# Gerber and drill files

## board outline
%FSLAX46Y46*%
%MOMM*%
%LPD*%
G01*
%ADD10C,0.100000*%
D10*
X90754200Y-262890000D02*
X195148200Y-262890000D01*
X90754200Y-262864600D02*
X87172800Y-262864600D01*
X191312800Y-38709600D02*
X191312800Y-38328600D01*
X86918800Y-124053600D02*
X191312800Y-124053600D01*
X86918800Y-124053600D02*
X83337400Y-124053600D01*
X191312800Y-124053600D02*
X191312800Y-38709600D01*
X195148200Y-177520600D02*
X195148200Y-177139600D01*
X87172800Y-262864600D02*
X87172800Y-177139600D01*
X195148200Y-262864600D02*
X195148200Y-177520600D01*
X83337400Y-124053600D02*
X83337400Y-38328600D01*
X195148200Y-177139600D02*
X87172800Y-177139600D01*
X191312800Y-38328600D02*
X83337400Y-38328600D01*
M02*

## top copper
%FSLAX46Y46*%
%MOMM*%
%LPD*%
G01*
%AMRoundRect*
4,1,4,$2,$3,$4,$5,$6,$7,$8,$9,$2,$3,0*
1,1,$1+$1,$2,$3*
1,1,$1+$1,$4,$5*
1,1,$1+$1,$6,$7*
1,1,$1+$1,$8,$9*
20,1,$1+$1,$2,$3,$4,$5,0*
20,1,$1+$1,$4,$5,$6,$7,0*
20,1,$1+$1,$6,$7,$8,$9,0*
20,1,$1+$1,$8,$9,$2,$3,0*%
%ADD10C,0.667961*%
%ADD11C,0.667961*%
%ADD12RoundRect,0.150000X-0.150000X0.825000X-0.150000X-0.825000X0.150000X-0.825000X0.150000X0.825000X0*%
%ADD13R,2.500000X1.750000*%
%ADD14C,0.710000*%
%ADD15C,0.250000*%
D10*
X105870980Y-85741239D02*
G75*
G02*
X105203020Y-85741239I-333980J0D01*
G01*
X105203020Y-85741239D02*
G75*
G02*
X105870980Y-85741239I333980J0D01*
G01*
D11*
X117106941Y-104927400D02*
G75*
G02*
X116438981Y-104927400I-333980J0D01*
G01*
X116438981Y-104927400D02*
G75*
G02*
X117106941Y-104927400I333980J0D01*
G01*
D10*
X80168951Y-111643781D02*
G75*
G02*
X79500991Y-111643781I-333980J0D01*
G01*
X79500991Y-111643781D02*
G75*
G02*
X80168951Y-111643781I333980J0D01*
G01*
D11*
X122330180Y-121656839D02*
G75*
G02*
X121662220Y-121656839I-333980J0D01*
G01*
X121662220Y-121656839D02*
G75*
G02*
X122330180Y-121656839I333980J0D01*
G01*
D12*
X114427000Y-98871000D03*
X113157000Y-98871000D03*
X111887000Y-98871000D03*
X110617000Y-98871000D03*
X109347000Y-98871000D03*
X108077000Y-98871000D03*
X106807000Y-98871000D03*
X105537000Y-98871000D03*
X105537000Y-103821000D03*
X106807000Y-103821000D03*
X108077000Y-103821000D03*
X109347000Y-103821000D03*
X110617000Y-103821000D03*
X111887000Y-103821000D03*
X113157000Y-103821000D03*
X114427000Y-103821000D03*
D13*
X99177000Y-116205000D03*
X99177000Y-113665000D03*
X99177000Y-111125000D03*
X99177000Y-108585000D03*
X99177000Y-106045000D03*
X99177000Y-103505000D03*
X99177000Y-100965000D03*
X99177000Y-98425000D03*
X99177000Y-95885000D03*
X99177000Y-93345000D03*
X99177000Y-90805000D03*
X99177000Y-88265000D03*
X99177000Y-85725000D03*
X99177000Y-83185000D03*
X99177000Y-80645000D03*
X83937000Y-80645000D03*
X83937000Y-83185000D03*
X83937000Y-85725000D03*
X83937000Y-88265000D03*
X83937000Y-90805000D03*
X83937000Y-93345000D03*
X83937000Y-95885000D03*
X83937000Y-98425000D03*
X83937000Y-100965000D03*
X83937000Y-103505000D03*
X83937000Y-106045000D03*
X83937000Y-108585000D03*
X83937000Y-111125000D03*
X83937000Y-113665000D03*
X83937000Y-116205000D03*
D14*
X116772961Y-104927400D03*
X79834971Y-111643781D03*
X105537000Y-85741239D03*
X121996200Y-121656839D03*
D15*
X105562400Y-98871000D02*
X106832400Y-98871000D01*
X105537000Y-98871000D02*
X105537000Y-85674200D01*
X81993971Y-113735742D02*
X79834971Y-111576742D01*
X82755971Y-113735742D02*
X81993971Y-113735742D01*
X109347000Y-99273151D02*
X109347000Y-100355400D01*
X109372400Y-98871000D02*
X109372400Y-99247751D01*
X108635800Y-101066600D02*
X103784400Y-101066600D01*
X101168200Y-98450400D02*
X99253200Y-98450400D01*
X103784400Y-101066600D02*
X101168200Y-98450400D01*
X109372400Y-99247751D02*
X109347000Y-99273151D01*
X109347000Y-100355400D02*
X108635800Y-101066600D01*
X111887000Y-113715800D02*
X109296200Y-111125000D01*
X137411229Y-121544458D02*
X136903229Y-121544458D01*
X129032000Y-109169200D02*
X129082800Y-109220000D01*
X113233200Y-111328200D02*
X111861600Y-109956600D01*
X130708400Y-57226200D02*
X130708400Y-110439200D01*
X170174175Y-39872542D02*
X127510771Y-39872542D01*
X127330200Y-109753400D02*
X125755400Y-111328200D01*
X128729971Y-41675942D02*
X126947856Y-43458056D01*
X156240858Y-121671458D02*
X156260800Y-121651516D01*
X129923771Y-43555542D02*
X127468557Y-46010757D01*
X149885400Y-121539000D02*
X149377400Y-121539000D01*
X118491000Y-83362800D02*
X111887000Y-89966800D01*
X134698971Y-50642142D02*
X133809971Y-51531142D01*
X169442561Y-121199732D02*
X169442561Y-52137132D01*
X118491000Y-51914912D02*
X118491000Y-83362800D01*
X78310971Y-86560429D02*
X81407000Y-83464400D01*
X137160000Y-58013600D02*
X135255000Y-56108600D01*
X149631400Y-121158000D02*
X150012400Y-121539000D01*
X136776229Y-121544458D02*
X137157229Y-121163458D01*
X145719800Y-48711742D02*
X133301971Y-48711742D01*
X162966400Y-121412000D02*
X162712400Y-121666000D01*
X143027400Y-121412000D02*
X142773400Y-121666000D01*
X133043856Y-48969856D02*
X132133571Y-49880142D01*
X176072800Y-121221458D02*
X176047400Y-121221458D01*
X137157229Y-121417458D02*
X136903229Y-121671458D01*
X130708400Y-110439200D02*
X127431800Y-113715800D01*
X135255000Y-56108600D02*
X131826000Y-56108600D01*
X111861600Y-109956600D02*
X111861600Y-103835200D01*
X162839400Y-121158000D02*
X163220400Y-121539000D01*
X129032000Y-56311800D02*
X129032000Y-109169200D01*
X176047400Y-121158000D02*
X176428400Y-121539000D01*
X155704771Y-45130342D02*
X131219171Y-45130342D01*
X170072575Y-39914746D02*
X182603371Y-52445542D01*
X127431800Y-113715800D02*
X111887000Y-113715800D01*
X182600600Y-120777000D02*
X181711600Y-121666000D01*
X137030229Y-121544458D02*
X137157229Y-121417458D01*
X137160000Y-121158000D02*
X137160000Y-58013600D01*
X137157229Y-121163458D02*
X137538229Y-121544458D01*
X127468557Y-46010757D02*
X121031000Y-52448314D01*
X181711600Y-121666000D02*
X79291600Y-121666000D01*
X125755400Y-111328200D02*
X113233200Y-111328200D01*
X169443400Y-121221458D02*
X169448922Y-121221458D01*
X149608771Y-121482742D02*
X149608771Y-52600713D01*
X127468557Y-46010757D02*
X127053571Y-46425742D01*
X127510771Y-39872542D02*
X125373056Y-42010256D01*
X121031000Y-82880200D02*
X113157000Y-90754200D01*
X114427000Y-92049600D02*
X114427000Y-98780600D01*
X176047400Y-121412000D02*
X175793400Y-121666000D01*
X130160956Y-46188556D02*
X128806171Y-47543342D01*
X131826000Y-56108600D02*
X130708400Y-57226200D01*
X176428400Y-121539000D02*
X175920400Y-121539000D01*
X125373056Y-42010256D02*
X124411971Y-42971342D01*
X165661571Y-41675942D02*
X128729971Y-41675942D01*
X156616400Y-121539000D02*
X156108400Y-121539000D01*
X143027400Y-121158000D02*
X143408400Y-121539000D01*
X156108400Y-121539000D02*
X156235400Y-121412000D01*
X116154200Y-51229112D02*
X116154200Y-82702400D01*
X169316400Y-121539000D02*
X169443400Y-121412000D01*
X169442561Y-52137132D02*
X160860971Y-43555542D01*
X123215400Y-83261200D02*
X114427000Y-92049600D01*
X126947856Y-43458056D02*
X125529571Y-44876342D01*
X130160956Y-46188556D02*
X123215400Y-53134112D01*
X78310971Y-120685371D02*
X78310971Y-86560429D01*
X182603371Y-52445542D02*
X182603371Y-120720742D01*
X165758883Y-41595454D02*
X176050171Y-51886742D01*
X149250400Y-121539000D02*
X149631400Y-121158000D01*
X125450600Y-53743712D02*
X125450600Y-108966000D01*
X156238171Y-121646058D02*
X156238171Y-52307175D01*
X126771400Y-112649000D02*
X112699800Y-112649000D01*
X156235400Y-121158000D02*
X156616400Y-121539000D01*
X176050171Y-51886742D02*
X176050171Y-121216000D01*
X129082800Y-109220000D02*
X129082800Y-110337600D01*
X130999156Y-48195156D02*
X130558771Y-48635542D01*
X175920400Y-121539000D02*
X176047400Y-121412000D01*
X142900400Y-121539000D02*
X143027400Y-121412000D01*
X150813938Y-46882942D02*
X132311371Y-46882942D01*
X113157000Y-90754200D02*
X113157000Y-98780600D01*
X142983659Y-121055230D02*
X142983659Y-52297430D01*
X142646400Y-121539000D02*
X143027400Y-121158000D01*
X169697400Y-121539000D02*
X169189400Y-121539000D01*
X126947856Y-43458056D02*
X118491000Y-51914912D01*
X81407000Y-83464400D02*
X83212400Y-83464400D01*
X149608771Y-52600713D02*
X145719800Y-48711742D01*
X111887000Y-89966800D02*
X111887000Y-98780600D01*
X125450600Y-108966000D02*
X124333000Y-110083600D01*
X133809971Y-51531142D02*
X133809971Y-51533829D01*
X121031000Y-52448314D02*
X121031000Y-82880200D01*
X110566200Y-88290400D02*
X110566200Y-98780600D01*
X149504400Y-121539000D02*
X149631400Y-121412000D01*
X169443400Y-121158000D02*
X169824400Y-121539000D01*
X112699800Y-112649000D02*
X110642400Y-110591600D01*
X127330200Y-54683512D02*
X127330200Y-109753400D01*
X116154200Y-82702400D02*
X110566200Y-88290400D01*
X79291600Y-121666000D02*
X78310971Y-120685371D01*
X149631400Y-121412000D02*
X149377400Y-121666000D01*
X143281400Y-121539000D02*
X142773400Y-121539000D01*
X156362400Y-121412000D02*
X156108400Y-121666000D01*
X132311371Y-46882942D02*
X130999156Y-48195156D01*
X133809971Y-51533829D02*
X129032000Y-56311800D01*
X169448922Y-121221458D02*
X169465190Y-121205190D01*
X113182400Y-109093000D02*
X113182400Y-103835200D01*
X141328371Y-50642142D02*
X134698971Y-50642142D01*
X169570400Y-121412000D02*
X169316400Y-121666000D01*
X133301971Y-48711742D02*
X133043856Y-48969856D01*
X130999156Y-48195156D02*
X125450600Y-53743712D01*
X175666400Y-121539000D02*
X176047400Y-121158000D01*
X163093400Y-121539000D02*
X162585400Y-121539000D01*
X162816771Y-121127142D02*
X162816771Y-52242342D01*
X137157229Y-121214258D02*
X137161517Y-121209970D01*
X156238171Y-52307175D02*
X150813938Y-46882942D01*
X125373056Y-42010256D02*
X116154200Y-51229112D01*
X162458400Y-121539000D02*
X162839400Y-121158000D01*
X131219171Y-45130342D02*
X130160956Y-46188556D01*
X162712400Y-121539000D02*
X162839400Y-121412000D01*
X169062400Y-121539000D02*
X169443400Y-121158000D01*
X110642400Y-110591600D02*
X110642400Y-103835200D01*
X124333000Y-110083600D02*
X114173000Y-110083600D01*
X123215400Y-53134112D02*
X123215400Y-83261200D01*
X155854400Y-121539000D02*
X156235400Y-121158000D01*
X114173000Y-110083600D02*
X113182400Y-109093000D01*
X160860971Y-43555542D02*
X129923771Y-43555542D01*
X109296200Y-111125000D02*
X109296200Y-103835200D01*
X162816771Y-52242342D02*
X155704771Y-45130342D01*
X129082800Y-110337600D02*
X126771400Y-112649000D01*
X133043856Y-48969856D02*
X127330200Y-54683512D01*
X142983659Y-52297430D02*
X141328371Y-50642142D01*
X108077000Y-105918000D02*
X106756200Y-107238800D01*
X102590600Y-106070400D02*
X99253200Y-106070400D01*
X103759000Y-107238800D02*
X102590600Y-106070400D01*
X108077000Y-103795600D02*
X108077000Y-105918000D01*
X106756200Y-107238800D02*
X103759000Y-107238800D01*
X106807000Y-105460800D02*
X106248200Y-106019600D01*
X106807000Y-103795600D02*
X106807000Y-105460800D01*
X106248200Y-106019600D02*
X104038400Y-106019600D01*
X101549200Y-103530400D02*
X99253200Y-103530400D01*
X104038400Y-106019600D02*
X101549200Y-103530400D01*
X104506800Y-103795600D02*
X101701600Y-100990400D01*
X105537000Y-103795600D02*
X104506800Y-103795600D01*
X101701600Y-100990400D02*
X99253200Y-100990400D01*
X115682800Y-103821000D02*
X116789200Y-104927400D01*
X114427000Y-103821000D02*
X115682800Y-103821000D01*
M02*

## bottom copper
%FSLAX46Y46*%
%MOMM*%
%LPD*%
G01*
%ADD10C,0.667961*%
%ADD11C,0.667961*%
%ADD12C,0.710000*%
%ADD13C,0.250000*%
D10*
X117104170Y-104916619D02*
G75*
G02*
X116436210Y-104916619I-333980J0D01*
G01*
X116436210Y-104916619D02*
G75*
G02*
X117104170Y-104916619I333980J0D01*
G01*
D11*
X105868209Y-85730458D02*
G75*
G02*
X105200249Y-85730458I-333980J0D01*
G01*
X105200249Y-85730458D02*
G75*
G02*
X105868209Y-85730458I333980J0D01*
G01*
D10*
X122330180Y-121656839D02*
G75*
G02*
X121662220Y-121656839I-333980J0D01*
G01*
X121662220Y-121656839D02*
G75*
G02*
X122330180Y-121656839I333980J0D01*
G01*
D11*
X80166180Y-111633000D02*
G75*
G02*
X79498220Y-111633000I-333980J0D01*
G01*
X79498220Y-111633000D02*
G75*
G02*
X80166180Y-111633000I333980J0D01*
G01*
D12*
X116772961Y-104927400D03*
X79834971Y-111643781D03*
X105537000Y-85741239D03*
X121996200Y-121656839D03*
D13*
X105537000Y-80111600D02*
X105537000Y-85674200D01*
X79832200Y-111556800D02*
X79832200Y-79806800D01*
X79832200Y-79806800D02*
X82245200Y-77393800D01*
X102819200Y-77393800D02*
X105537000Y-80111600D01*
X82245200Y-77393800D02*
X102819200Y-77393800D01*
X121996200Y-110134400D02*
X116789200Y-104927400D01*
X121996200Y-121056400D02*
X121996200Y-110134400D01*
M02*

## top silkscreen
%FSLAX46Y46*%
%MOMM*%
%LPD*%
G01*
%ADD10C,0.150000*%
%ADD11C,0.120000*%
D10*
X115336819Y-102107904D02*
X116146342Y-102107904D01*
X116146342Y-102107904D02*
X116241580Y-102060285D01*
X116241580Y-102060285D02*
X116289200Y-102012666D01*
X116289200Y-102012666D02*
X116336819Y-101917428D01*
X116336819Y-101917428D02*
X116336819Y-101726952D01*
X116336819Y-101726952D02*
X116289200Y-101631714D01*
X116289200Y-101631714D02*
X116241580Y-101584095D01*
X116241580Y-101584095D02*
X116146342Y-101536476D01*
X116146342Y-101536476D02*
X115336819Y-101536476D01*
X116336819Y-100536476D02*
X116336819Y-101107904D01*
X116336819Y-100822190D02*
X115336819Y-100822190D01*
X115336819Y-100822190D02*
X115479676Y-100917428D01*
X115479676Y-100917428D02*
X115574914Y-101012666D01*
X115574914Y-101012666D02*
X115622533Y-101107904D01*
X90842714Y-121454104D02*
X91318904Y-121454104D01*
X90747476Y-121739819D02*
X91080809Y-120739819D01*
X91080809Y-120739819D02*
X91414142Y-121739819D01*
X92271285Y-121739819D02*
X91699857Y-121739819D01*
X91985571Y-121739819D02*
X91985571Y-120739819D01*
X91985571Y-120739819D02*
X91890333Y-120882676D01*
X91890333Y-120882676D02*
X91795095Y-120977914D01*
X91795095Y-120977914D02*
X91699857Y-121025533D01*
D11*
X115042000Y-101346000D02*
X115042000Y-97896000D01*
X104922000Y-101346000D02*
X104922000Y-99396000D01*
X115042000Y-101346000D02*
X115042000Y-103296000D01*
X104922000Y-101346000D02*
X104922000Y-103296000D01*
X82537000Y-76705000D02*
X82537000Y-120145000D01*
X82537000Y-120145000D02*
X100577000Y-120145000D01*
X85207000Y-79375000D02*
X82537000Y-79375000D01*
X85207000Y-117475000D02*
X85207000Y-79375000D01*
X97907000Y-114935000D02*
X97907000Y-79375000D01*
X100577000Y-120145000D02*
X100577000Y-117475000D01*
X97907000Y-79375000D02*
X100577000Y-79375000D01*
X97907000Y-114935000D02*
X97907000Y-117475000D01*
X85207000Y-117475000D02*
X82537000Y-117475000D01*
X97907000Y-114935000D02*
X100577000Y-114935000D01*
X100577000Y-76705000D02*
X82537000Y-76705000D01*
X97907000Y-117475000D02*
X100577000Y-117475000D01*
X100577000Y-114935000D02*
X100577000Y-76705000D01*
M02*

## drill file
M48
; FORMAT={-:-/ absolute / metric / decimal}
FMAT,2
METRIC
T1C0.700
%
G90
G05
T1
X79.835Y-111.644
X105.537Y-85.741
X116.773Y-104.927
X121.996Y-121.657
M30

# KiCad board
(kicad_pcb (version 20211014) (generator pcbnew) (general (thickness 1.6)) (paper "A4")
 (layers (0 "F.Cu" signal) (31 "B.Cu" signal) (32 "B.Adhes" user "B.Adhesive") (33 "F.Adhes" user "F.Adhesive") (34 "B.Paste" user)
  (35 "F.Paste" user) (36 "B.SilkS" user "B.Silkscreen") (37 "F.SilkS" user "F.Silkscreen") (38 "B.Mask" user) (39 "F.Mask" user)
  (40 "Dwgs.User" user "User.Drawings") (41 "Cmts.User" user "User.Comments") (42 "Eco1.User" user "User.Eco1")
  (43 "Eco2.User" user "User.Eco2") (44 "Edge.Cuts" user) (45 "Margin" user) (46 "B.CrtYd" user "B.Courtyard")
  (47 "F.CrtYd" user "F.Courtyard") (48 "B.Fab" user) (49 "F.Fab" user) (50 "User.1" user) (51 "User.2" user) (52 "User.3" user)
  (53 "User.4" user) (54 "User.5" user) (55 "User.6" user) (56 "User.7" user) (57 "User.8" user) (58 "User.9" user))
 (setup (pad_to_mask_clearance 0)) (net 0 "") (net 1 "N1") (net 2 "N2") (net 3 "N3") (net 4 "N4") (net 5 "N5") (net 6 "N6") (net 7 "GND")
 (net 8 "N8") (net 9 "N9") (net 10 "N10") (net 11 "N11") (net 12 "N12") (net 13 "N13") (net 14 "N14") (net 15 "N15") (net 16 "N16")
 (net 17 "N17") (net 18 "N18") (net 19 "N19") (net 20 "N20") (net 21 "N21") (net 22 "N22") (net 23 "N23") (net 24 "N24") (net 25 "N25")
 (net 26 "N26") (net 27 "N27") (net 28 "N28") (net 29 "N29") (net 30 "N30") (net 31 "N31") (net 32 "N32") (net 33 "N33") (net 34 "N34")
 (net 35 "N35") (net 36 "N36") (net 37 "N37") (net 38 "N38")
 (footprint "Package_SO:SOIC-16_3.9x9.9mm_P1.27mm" (layer "F.Cu") (at 109.982 101.346 -90)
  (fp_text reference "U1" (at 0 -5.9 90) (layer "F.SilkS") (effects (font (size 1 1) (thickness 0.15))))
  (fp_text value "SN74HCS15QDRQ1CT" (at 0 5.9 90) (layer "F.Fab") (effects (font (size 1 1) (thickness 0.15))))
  (fp_line (start 0 -5.06) (end -3.45 -5.06) (layer "F.SilkS") (width 0.12))
  (fp_line (start 0 5.06) (end -1.95 5.06) (layer "F.SilkS") (width 0.12))
  (fp_line (start 0 -5.06) (end 1.95 -5.06) (layer "F.SilkS") (width 0.12))
  (fp_line (start 0 5.06) (end 1.95 5.06) (layer "F.SilkS") (width 0.12))
  (pad "1" smd roundrect (at -2.475 -4.445 270) (size 1.95 0.6) (layers "F.Cu" "F.Paste" "F.Mask") (roundrect_rratio 0.25) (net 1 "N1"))
  (pad "2" smd roundrect (at -2.475 -3.175 270) (size 1.95 0.6) (layers "F.Cu" "F.Paste" "F.Mask") (roundrect_rratio 0.25) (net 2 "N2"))
  (pad "3" smd roundrect (at -2.475 -1.905 270) (size 1.95 0.6) (layers "F.Cu" "F.Paste" "F.Mask") (roundrect_rratio 0.25) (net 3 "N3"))
  (pad "4" smd roundrect (at -2.475 -0.635 270) (size 1.95 0.6) (layers "F.Cu" "F.Paste" "F.Mask") (roundrect_rratio 0.25) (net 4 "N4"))
  (pad "5" smd roundrect (at -2.475 0.635 270) (size 1.95 0.6) (layers "F.Cu" "F.Paste" "F.Mask") (roundrect_rratio 0.25) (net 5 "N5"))
  (pad "6" smd roundrect (at -2.475 1.905 270) (size 1.95 0.6) (layers "F.Cu" "F.Paste" "F.Mask") (roundrect_rratio 0.25) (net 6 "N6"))
  (pad "7" smd roundrect (at -2.475 3.175 270) (size 1.95 0.6) (layers "F.Cu" "F.Paste" "F.Mask") (roundrect_rratio 0.25) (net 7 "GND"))
  (pad "8" smd roundrect (at -2.475 4.445 270) (size 1.95 0.6) (layers "F.Cu" "F.Paste" "F.Mask") (roundrect_rratio 0.25) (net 7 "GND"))
  (pad "9" smd roundrect (at 2.475 4.445 270) (size 1.95 0.6) (layers "F.Cu" "F.Paste" "F.Mask") (roundrect_rratio 0.25) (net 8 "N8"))
  (pad "10" smd roundrect (at 2.475 3.175 270) (size 1.95 0.6) (layers "F.Cu" "F.Paste" "F.Mask") (roundrect_rratio 0.25) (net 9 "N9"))
  (pad "11" smd roundrect (at 2.475 1.905 270) (size 1.95 0.6) (layers "F.Cu" "F.Paste" "F.Mask") (roundrect_rratio 0.25) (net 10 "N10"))
  (pad "12" smd roundrect (at 2.475 0.635 270) (size 1.95 0.6) (layers "F.Cu" "F.Paste" "F.Mask") (roundrect_rratio 0.25) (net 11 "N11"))
  (pad "13" smd roundrect (at 2.475 -0.635 270) (size 1.95 0.6) (layers "F.Cu" "F.Paste" "F.Mask") (roundrect_rratio 0.25) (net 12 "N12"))
  (pad "14" smd roundrect (at 2.475 -1.905 270) (size 1.95 0.6) (layers "F.Cu" "F.Paste" "F.Mask") (roundrect_rratio 0.25) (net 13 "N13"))
  (pad "15" smd roundrect (at 2.475 -3.175 270) (size 1.95 0.6) (layers "F.Cu" "F.Paste" "F.Mask") (roundrect_rratio 0.25) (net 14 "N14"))
  (pad "16" smd roundrect (at 2.475 -4.445 270) (size 1.95 0.6) (layers "F.Cu" "F.Paste" "F.Mask") (roundrect_rratio 0.25) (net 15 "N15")))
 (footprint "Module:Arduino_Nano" (layer "F.Cu") (at 99.177 116.205 180)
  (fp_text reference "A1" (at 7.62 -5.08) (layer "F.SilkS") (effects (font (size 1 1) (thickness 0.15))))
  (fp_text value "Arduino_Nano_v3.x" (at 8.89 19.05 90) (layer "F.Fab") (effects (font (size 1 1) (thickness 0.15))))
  (fp_line (start 16.64 39.5) (end 16.64 -3.94) (layer "F.SilkS") (width 0.12))
  (fp_line (start 16.64 -3.94) (end -1.4 -3.94) (layer "F.SilkS") (width 0.12))
  (fp_line (start 13.97 36.83) (end 16.64 36.83) (layer "F.SilkS") (width 0.12))
  (fp_line (start 13.97 -1.27) (end 13.97 36.83) (layer "F.SilkS") (width 0.12))
  (fp_line (start 1.27 1.27) (end 1.27 36.83) (layer "F.SilkS") (width 0.12))
  (fp_line (start -1.4 -3.94) (end -1.4 -1.27) (layer "F.SilkS") (width 0.12))
  (fp_line (start 1.27 36.83) (end -1.4 36.83) (layer "F.SilkS") (width 0.12))
  (fp_line (start 1.27 1.27) (end 1.27 -1.27) (layer "F.SilkS") (width 0.12))
  (fp_line (start 13.97 -1.27) (end 16.64 -1.27) (layer "F.SilkS") (width 0.12))
  (fp_line (start 1.27 1.27) (end -1.4 1.27) (layer "F.SilkS") (width 0.12))
  (fp_line (start -1.4 39.5) (end 16.64 39.5) (layer "F.SilkS") (width 0.12))
  (fp_line (start 1.27 -1.27) (end -1.4 -1.27) (layer "F.SilkS") (width 0.12))
  (fp_line (start -1.4 1.27) (end -1.4 39.5) (layer "F.SilkS") (width 0.12))
  (pad "1" smd rect (at 0 0 180) (size 2.5 1.75) (layers "F.Cu" "F.Paste" "F.Mask") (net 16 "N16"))
  (pad "2" smd rect (at 0 2.54 180) (size 2.5 1.75) (layers "F.Cu" "F.Paste" "F.Mask") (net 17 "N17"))
  (pad "3" smd rect (at 0 5.08 180) (size 2.5 1.75) (layers "F.Cu" "F.Paste" "F.Mask") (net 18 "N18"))
  (pad "4" smd rect (at 0 7.62 180) (size 2.5 1.75) (layers "F.Cu" "F.Paste" "F.Mask") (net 7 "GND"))
  (pad "5" smd rect (at 0 10.16 180) (size 2.5 1.75) (layers "F.Cu" "F.Paste" "F.Mask") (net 10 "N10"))
  (pad "6" smd rect (at 0 12.7 180) (size 2.5 1.75) (layers "F.Cu" "F.Paste" "F.Mask") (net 9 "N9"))
  (pad "7" smd rect (at 0 15.24 180) (size 2.5 1.75) (layers "F.Cu" "F.Paste" "F.Mask") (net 8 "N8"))
  (pad "8" smd rect (at 0 17.78 180) (size 2.5 1.75) (layers "F.Cu" "F.Paste" "F.Mask") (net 5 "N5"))
  (pad "9" smd rect (at 0 20.32 180) (size 2.5 1.75) (layers "F.Cu" "F.Paste" "F.Mask") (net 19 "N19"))
  (pad "10" smd rect (at 0 22.86 180) (size 2.5 1.75) (layers "F.Cu" "F.Paste" "F.Mask") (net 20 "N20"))
  (pad "11" smd rect (at 0 25.4 180) (size 2.5 1.75) (layers "F.Cu" "F.Paste" "F.Mask") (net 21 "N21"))
  (pad "12" smd rect (at 0 27.94 180) (size 2.5 1.75) (layers "F.Cu" "F.Paste" "F.Mask") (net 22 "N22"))
  (pad "13" smd rect (at 0 30.48 180) (size 2.5 1.75) (layers "F.Cu" "F.Paste" "F.Mask") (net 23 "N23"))
  (pad "14" smd rect (at 0 33.02 180) (size 2.5 1.75) (layers "F.Cu" "F.Paste" "F.Mask") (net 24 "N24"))
  (pad "15" smd rect (at 0 35.56 180) (size 2.5 1.75) (layers "F.Cu" "F.Paste" "F.Mask") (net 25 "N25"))
  (pad "16" smd rect (at 15.24 35.56 180) (size 2.5 1.75) (layers "F.Cu" "F.Paste" "F.Mask") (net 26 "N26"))
  (pad "17" smd rect (at 15.24 33.02 180) (size 2.5 1.75) (layers "F.Cu" "F.Paste" "F.Mask") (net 15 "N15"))
  (pad "18" smd rect (at 15.24 30.48 180) (size 2.5 1.75) (layers "F.Cu" "F.Paste" "F.Mask") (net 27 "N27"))
  (pad "19" smd rect (at 15.24 27.94 180) (size 2.5 1.75) (layers "F.Cu" "F.Paste" "F.Mask") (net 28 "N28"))
  (pad "20" smd rect (at 15.24 25.4 180) (size 2.5 1.75) (layers "F.Cu" "F.Paste" "F.Mask") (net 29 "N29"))
  (pad "21" smd rect (at 15.24 22.86 180) (size 2.5 1.75) (layers "F.Cu" "F.Paste" "F.Mask") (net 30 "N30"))
  (pad "22" smd rect (at 15.24 20.32 180) (size 2.5 1.75) (layers "F.Cu" "F.Paste" "F.Mask") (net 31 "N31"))
  (pad "23" smd rect (at 15.24 17.78 180) (size 2.5 1.75) (layers "F.Cu" "F.Paste" "F.Mask") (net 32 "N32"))
  (pad "24" smd rect (at 15.24 15.24 180) (size 2.5 1.75) (layers "F.Cu" "F.Paste" "F.Mask") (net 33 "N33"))
  (pad "25" smd rect (at 15.24 12.7 180) (size 2.5 1.75) (layers "F.Cu" "F.Paste" "F.Mask") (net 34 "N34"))
  (pad "26" smd rect (at 15.24 10.16 180) (size 2.5 1.75) (layers "F.Cu" "F.Paste" "F.Mask") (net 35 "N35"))
  (pad "27" smd rect (at 15.24 7.62 180) (size 2.5 1.75) (layers "F.Cu" "F.Paste" "F.Mask") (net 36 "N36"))
  (pad "28" smd rect (at 15.24 5.08 180) (size 2.5 1.75) (layers "F.Cu" "F.Paste" "F.Mask") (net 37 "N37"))
  (pad "29" smd rect (at 15.24 2.54 180) (size 2.5 1.75) (layers "F.Cu" "F.Paste" "F.Mask") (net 7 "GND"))
  (pad "30" smd rect (at 15.24 0 180) (size 2.5 1.75) (layers "F.Cu" "F.Paste" "F.Mask") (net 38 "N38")))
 (gr_circle (center 105.537 85.741239) (end 106.104961 85.741239) (layer "F.Cu") (width 0.2) (fill solid))
 (gr_circle (center 116.772961 104.9274) (end 117.340922 104.9274) (layer "F.Cu") (width 0.2) (fill solid))
 (gr_circle (center 79.834971 111.643781) (end 80.402932 111.643781) (layer "F.Cu") (width 0.2) (fill solid))
 (gr_circle (center 121.9962 121.656839) (end 122.564161 121.656839) (layer "F.Cu") (width 0.2) (fill solid))
 (gr_circle (center 116.77019 104.916619) (end 117.338151 104.916619) (layer "B.Cu") (width 0.2) (fill solid))
 (gr_circle (center 105.534229 85.730458) (end 106.10219 85.730458) (layer "B.Cu") (width 0.2) (fill solid))
 (gr_circle (center 121.9962 121.656839) (end 122.564161 121.656839) (layer "B.Cu") (width 0.2) (fill solid))
 (gr_circle (center 79.8322 111.633) (end 80.400161 111.633) (layer "B.Cu") (width 0.2) (fill solid))
 (gr_line (start 90.7542 262.89) (end 195.1482 262.89) (layer "Edge.Cuts") (width 0.1))
 (gr_line (start 90.7542 262.8646) (end 87.1728 262.8646) (layer "Edge.Cuts") (width 0.1))
 (gr_line (start 191.3128 38.7096) (end 191.3128 38.3286) (layer "Edge.Cuts") (width 0.1))
 (gr_line (start 86.9188 124.0536) (end 191.3128 124.0536) (layer "Edge.Cuts") (width 0.1))
 (gr_line (start 86.9188 124.0536) (end 83.3374 124.0536) (layer "Edge.Cuts") (width 0.1))
 (gr_line (start 191.3128 124.0536) (end 191.3128 38.7096) (layer "Edge.Cuts") (width 0.1))
 (gr_line (start 195.1482 177.5206) (end 195.1482 177.1396) (layer "Edge.Cuts") (width 0.1))
 (gr_line (start 87.1728 262.8646) (end 87.1728 177.1396) (layer "Edge.Cuts") (width 0.1))
 (gr_line (start 195.1482 262.8646) (end 195.1482 177.5206) (layer "Edge.Cuts") (width 0.1))
 (gr_line (start 83.3374 124.0536) (end 83.3374 38.3286) (layer "Edge.Cuts") (width 0.1))
 (gr_line (start 195.1482 177.1396) (end 87.1728 177.1396) (layer "Edge.Cuts") (width 0.1))
 (gr_line (start 191.3128 38.3286) (end 83.3374 38.3286) (layer "Edge.Cuts") (width 0.1))
 (via (at 116.772961 104.9274) (size 0.71) (drill 0.7) (layers "F.Cu" "B.Cu") (free) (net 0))
 (via (at 79.834971 111.643781) (size 0.71) (drill 0.7) (layers "F.Cu" "B.Cu") (free) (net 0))
 (via (at 105.537 85.741239) (size 0.71) (drill 0.7) (layers "F.Cu" "B.Cu") (free) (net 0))
 (via (at 121.9962 121.656839) (size 0.71) (drill 0.7) (layers "F.Cu" "B.Cu") (free) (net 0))
 (segment (start 105.5624 98.871) (end 106.8324 98.871) (width 0.25) (layer "F.Cu") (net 7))
 (segment (start 105.537 98.871) (end 105.537 85.6742) (width 0.25) (layer "F.Cu") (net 7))
 (segment (start 81.993971 113.735742) (end 79.834971 111.576742) (width 0.25) (layer "F.Cu") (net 7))
 (segment (start 82.755971 113.735742) (end 81.993971 113.735742) (width 0.25) (layer "F.Cu") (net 7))
 (segment (start 105.537 80.1116) (end 105.537 85.6742) (width 0.25) (layer "B.Cu") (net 7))
 (segment (start 79.8322 111.5568) (end 79.8322 79.8068) (width 0.25) (layer "B.Cu") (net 7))
 (segment (start 79.8322 79.8068) (end 82.2452 77.3938) (width 0.25) (layer "B.Cu") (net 7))
 (segment (start 102.8192 77.3938) (end 105.537 80.1116) (width 0.25) (layer "B.Cu") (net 7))
 (segment (start 82.2452 77.3938) (end 102.8192 77.3938) (width 0.25) (layer "B.Cu") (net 7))
 (segment (start 109.347 99.273151) (end 109.347 100.3554) (width 0.25) (layer "F.Cu") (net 5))
 (segment (start 109.3724 98.871) (end 109.3724 99.247751) (width 0.25) (layer "F.Cu") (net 5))
 (segment (start 108.6358 101.0666) (end 103.7844 101.0666) (width 0.25) (layer "F.Cu") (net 5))
 (segment (start 101.1682 98.4504) (end 99.2532 98.4504) (width 0.25) (layer "F.Cu") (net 5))
 (segment (start 103.7844 101.0666) (end 101.1682 98.4504) (width 0.25) (layer "F.Cu") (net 5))
 (segment (start 109.3724 99.247751) (end 109.347 99.273151) (width 0.25) (layer "F.Cu") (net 5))
 (segment (start 109.347 100.3554) (end 108.6358 101.0666) (width 0.25) (layer "F.Cu") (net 5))
 (segment (start 111.887 113.7158) (end 109.2962 111.125) (width 0.25) (layer "F.Cu") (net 2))
 (segment (start 137.411229 121.544458) (end 136.903229 121.544458) (width 0.25) (layer "F.Cu") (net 2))
 (segment (start 129.032 109.1692) (end 129.0828 109.22) (width 0.25) (layer "F.Cu") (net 2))
 (segment (start 113.2332 111.3282) (end 111.8616 109.9566) (width 0.25) (layer "F.Cu") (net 2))
 (segment (start 130.7084 57.2262) (end 130.7084 110.4392) (width 0.25) (layer "F.Cu") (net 2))
 (segment (start 170.174175 39.872542) (end 127.510771 39.872542) (width 0.25) (layer "F.Cu") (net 2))
 (segment (start 127.3302 109.7534) (end 125.7554 111.3282) (width 0.25) (layer "F.Cu") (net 2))
 (segment (start 128.729971 41.675942) (end 126.947856 43.458056) (width 0.25) (layer "F.Cu") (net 2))
 (segment (start 156.240858 121.671458) (end 156.2608 121.651516) (width 0.25) (layer "F.Cu") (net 2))
 (segment (start 129.923771 43.555542) (end 127.468557 46.010757) (width 0.25) (layer "F.Cu") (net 2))
 (segment (start 149.8854 121.539) (end 149.3774 121.539) (width 0.25) (layer "F.Cu") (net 2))
 (segment (start 118.491 83.3628) (end 111.887 89.9668) (width 0.25) (layer "F.Cu") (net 2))
 (segment (start 134.698971 50.642142) (end 133.809971 51.531142) (width 0.25) (layer "F.Cu") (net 2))
 (segment (start 169.442561 121.199732) (end 169.442561 52.137132) (width 0.25) (layer "F.Cu") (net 2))
 (segment (start 118.491 51.914912) (end 118.491 83.3628) (width 0.25) (layer "F.Cu") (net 2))
 (segment (start 78.310971 86.560429) (end 81.407 83.4644) (width 0.25) (layer "F.Cu") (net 2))
 (segment (start 137.16 58.0136) (end 135.255 56.1086) (width 0.25) (layer "F.Cu") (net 2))
 (segment (start 149.6314 121.158) (end 150.0124 121.539) (width 0.25) (layer "F.Cu") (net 2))
 (segment (start 136.776229 121.544458) (end 137.157229 121.163458) (width 0.25) (layer "F.Cu") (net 2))
 (segment (start 145.7198 48.711742) (end 133.301971 48.711742) (width 0.25) (layer "F.Cu") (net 2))
 (segment (start 162.9664 121.412) (end 162.7124 121.666) (width 0.25) (layer "F.Cu") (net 2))
 (segment (start 143.0274 121.412) (end 142.7734 121.666) (width 0.25) (layer "F.Cu") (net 2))
 (segment (start 133.043856 48.969856) (end 132.133571 49.880142) (width 0.25) (layer "F.Cu") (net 2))
 (segment (start 176.0728 121.221458) (end 176.0474 121.221458) (width 0.25) (layer "F.Cu") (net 2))
 (segment (start 137.157229 121.417458) (end 136.903229 121.671458) (width 0.25) (layer "F.Cu") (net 2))
 (segment (start 130.7084 110.4392) (end 127.4318 113.7158) (width 0.25) (layer "F.Cu") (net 2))
 (segment (start 135.255 56.1086) (end 131.826 56.1086) (width 0.25) (layer "F.Cu") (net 2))
 (segment (start 111.8616 109.9566) (end 111.8616 103.8352) (width 0.25) (layer "F.Cu") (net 2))
 (segment (start 162.8394 121.158) (end 163.2204 121.539) (width 0.25) (layer "F.Cu") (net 2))
 (segment (start 129.032 56.3118) (end 129.032 109.1692) (width 0.25) (layer "F.Cu") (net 2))
 (segment (start 176.0474 121.158) (end 176.4284 121.539) (width 0.25) (layer "F.Cu") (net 2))
 (segment (start 155.704771 45.130342) (end 131.219171 45.130342) (width 0.25) (layer "F.Cu") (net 2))
 (segment (start 170.072575 39.914746) (end 182.603371 52.445542) (width 0.25) (layer "F.Cu") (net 2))
 (segment (start 127.4318 113.7158) (end 111.887 113.7158) (width 0.25) (layer "F.Cu") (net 2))
 (segment (start 182.6006 120.777) (end 181.7116 121.666) (width 0.25) (layer "F.Cu") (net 2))
 (segment (start 137.030229 121.544458) (end 137.157229 121.417458) (width 0.25) (layer "F.Cu") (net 2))
 (segment (start 137.16 121.158) (end 137.16 58.0136) (width 0.25) (layer "F.Cu") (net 2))
 (segment (start 137.157229 121.163458) (end 137.538229 121.544458) (width 0.25) (layer "F.Cu") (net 2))
 (segment (start 127.468557 46.010757) (end 121.031 52.448314) (width 0.25) (layer "F.Cu") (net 2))
 (segment (start 181.7116 121.666) (end 79.2916 121.666) (width 0.25) (layer "F.Cu") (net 2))
 (segment (start 125.7554 111.3282) (end 113.2332 111.3282) (width 0.25) (layer "F.Cu") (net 2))
 (segment (start 169.4434 121.221458) (end 169.448922 121.221458) (width 0.25) (layer "F.Cu") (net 2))
 (segment (start 149.608771 121.482742) (end 149.608771 52.600713) (width 0.25) (layer "F.Cu") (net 2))
 (segment (start 127.468557 46.010757) (end 127.053571 46.425742) (width 0.25) (layer "F.Cu") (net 2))
 (segment (start 127.510771 39.872542) (end 125.373056 42.010256) (width 0.25) (layer "F.Cu") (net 2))
 (segment (start 121.031 82.8802) (end 113.157 90.7542) (width 0.25) (layer "F.Cu") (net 2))
 (segment (start 114.427 92.0496) (end 114.427 98.7806) (width 0.25) (layer "F.Cu") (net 2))
 (segment (start 176.0474 121.412) (end 175.7934 121.666) (width 0.25) (layer "F.Cu") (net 2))
 (segment (start 130.160956 46.188556) (end 128.806171 47.543342) (width 0.25) (layer "F.Cu") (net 2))
 (segment (start 131.826 56.1086) (end 130.7084 57.2262) (width 0.25) (layer "F.Cu") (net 2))
 (segment (start 176.4284 121.539) (end 175.9204 121.539) (width 0.25) (layer "F.Cu") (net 2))
 (segment (start 125.373056 42.010256) (end 124.411971 42.971342) (width 0.25) (layer "F.Cu") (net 2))
 (segment (start 165.661571 41.675942) (end 128.729971 41.675942) (width 0.25) (layer "F.Cu") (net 2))
 (segment (start 156.6164 121.539) (end 156.1084 121.539) (width 0.25) (layer "F.Cu") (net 2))
 (segment (start 143.0274 121.158) (end 143.4084 121.539) (width 0.25) (layer "F.Cu") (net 2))
 (segment (start 156.1084 121.539) (end 156.2354 121.412) (width 0.25) (layer "F.Cu") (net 2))
 (segment (start 116.1542 51.229112) (end 116.1542 82.7024) (width 0.25) (layer "F.Cu") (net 2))
 (segment (start 169.3164 121.539) (end 169.4434 121.412) (width 0.25) (layer "F.Cu") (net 2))
 (segment (start 169.442561 52.137132) (end 160.860971 43.555542) (width 0.25) (layer "F.Cu") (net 2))
 (segment (start 123.2154 83.2612) (end 114.427 92.0496) (width 0.25) (layer "F.Cu") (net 2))
 (segment (start 126.947856 43.458056) (end 125.529571 44.876342) (width 0.25) (layer "F.Cu") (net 2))
 (segment (start 130.160956 46.188556) (end 123.2154 53.134112) (width 0.25) (layer "F.Cu") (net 2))
 (segment (start 78.310971 120.685371) (end 78.310971 86.560429) (width 0.25) (layer "F.Cu") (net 2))
 (segment (start 182.603371 52.445542) (end 182.603371 120.720742) (width 0.25) (layer "F.Cu") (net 2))
 (segment (start 165.758883 41.595454) (end 176.050171 51.886742) (width 0.25) (layer "F.Cu") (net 2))
 (segment (start 149.2504 121.539) (end 149.6314 121.158) (width 0.25) (layer "F.Cu") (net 2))
 (segment (start 125.4506 53.743712) (end 125.4506 108.966) (width 0.25) (layer "F.Cu") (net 2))
 (segment (start 156.238171 121.646058) (end 156.238171 52.307175) (width 0.25) (layer "F.Cu") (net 2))
 (segment (start 126.7714 112.649) (end 112.6998 112.649) (width 0.25) (layer "F.Cu") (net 2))
 (segment (start 156.2354 121.158) (end 156.6164 121.539) (width 0.25) (layer "F.Cu") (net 2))
 (segment (start 176.050171 51.886742) (end 176.050171 121.216) (width 0.25) (layer "F.Cu") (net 2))
 (segment (start 129.0828 109.22) (end 129.0828 110.3376) (width 0.25) (layer "F.Cu") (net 2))
 (segment (start 130.999156 48.195156) (end 130.558771 48.635542) (width 0.25) (layer "F.Cu") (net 2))
 (segment (start 175.9204 121.539) (end 176.0474 121.412) (width 0.25) (layer "F.Cu") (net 2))
 (segment (start 142.9004 121.539) (end 143.0274 121.412) (width 0.25) (layer "F.Cu") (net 2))
 (segment (start 150.813938 46.882942) (end 132.311371 46.882942) (width 0.25) (layer "F.Cu") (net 2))
 (segment (start 113.157 90.7542) (end 113.157 98.7806) (width 0.25) (layer "F.Cu") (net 2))
 (segment (start 142.983659 121.05523) (end 142.983659 52.29743) (width 0.25) (layer "F.Cu") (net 2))
 (segment (start 142.6464 121.539) (end 143.0274 121.158) (width 0.25) (layer "F.Cu") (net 2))
 (segment (start 169.6974 121.539) (end 169.1894 121.539) (width 0.25) (layer "F.Cu") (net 2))
 (segment (start 126.947856 43.458056) (end 118.491 51.914912) (width 0.25) (layer "F.Cu") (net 2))
 (segment (start 81.407 83.4644) (end 83.2124 83.4644) (width 0.25) (layer "F.Cu") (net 2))
 (segment (start 149.608771 52.600713) (end 145.7198 48.711742) (width 0.25) (layer "F.Cu") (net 2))
 (segment (start 111.887 89.9668) (end 111.887 98.7806) (width 0.25) (layer "F.Cu") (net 2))
 (segment (start 125.4506 108.966) (end 124.333 110.0836) (width 0.25) (layer "F.Cu") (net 2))
 (segment (start 133.809971 51.531142) (end 133.809971 51.533829) (width 0.25) (layer "F.Cu") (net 2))
 (segment (start 121.031 52.448314) (end 121.031 82.8802) (width 0.25) (layer "F.Cu") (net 2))
 (segment (start 110.5662 88.2904) (end 110.5662 98.7806) (width 0.25) (layer "F.Cu") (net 2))
 (segment (start 149.5044 121.539) (end 149.6314 121.412) (width 0.25) (layer "F.Cu") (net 2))
 (segment (start 169.4434 121.158) (end 169.8244 121.539) (width 0.25) (layer "F.Cu") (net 2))
 (segment (start 112.6998 112.649) (end 110.6424 110.5916) (width 0.25) (layer "F.Cu") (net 2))
 (segment (start 127.3302 54.683512) (end 127.3302 109.7534) (width 0.25) (layer "F.Cu") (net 2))
 (segment (start 116.1542 82.7024) (end 110.5662 88.2904) (width 0.25) (layer "F.Cu") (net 2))
 (segment (start 79.2916 121.666) (end 78.310971 120.685371) (width 0.25) (layer "F.Cu") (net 2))
 (segment (start 149.6314 121.412) (end 149.3774 121.666) (width 0.25) (layer "F.Cu") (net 2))
 (segment (start 143.2814 121.539) (end 142.7734 121.539) (width 0.25) (layer "F.Cu") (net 2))
 (segment (start 156.3624 121.412) (end 156.1084 121.666) (width 0.25) (layer "F.Cu") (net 2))
 (segment (start 132.311371 46.882942) (end 130.999156 48.195156) (width 0.25) (layer "F.Cu") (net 2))
 (segment (start 133.809971 51.533829) (end 129.032 56.3118) (width 0.25) (layer "F.Cu") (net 2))
 (segment (start 169.448922 121.221458) (end 169.46519 121.20519) (width 0.25) (layer "F.Cu") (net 2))
 (segment (start 113.1824 109.093) (end 113.1824 103.8352) (width 0.25) (layer "F.Cu") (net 2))
 (segment (start 141.328371 50.642142) (end 134.698971 50.642142) (width 0.25) (layer "F.Cu") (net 2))
 (segment (start 169.5704 121.412) (end 169.3164 121.666) (width 0.25) (layer "F.Cu") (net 2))
 (segment (start 133.301971 48.711742) (end 133.043856 48.969856) (width 0.25) (layer "F.Cu") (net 2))
 (segment (start 130.999156 48.195156) (end 125.4506 53.743712) (width 0.25) (layer "F.Cu") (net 2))
 (segment (start 175.6664 121.539) (end 176.0474 121.158) (width 0.25) (layer "F.Cu") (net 2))
 (segment (start 163.0934 121.539) (end 162.5854 121.539) (width 0.25) (layer "F.Cu") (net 2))
 (segment (start 162.816771 121.127142) (end 162.816771 52.242342) (width 0.25) (layer "F.Cu") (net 2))
 (segment (start 137.157229 121.214258) (end 137.161517 121.20997) (width 0.25) (layer "F.Cu") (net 2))
 (segment (start 156.238171 52.307175) (end 150.813938 46.882942) (width 0.25) (layer "F.Cu") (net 2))
 (segment (start 125.373056 42.010256) (end 116.1542 51.229112) (width 0.25) (layer "F.Cu") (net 2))
 (segment (start 162.4584 121.539) (end 162.8394 121.158) (width 0.25) (layer "F.Cu") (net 2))
 (segment (start 131.219171 45.130342) (end 130.160956 46.188556) (width 0.25) (layer "F.Cu") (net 2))
 (segment (start 162.7124 121.539) (end 162.8394 121.412) (width 0.25) (layer "F.Cu") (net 2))
 (segment (start 169.0624 121.539) (end 169.4434 121.158) (width 0.25) (layer "F.Cu") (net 2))
 (segment (start 110.6424 110.5916) (end 110.6424 103.8352) (width 0.25) (layer "F.Cu") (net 2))
 (segment (start 124.333 110.0836) (end 114.173 110.0836) (width 0.25) (layer "F.Cu") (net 2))
 (segment (start 123.2154 53.134112) (end 123.2154 83.2612) (width 0.25) (layer "F.Cu") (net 2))
 (segment (start 155.8544 121.539) (end 156.2354 121.158) (width 0.25) (layer "F.Cu") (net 2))
 (segment (start 114.173 110.0836) (end 113.1824 109.093) (width 0.25) (layer "F.Cu") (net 2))
 (segment (start 160.860971 43.555542) (end 129.923771 43.555542) (width 0.25) (layer "F.Cu") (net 2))
 (segment (start 109.2962 111.125) (end 109.2962 103.8352) (width 0.25) (layer "F.Cu") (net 2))
 (segment (start 162.816771 52.242342) (end 155.704771 45.130342) (width 0.25) (layer "F.Cu") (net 2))
 (segment (start 129.0828 110.3376) (end 126.7714 112.649) (width 0.25) (layer "F.Cu") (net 2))
 (segment (start 133.043856 48.969856) (end 127.3302 54.683512) (width 0.25) (layer "F.Cu") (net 2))
 (segment (start 142.983659 52.29743) (end 141.328371 50.642142) (width 0.25) (layer "F.Cu") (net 2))
 (segment (start 108.077 105.918) (end 106.7562 107.2388) (width 0.25) (layer "F.Cu") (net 10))
 (segment (start 102.5906 106.0704) (end 99.2532 106.0704) (width 0.25) (layer "F.Cu") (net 10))
 (segment (start 103.759 107.2388) (end 102.5906 106.0704) (width 0.25) (layer "F.Cu") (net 10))
 (segment (start 108.077 103.7956) (end 108.077 105.918) (width 0.25) (layer "F.Cu") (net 10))
 (segment (start 106.7562 107.2388) (end 103.759 107.2388) (width 0.25) (layer "F.Cu") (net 10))
 (segment (start 106.807 105.4608) (end 106.2482 106.0196) (width 0.25) (layer "F.Cu") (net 9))
 (segment (start 106.807 103.7956) (end 106.807 105.4608) (width 0.25) (layer "F.Cu") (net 9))
 (segment (start 106.2482 106.0196) (end 104.0384 106.0196) (width 0.25) (layer "F.Cu") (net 9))
 (segment (start 101.5492 103.5304) (end 99.2532 103.5304) (width 0.25) (layer "F.Cu") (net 9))
 (segment (start 104.0384 106.0196) (end 101.5492 103.5304) (width 0.25) (layer "F.Cu") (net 9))
 (segment (start 104.5068 103.7956) (end 101.7016 100.9904) (width 0.25) (layer "F.Cu") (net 8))
 (segment (start 105.537 103.7956) (end 104.5068 103.7956) (width 0.25) (layer "F.Cu") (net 8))
 (segment (start 101.7016 100.9904) (end 99.2532 100.9904) (width 0.25) (layer "F.Cu") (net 8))
 (segment (start 115.6828 103.821) (end 116.7892 104.9274) (width 0.25) (layer "F.Cu") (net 15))
 (segment (start 114.427 103.821) (end 115.6828 103.821) (width 0.25) (layer "F.Cu") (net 15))
 (segment (start 121.9962 110.1344) (end 116.7892 104.9274) (width 0.25) (layer "B.Cu") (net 15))
 (segment (start 121.9962 121.0564) (end 121.9962 110.1344) (width 0.25) (layer "B.Cu") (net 15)))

